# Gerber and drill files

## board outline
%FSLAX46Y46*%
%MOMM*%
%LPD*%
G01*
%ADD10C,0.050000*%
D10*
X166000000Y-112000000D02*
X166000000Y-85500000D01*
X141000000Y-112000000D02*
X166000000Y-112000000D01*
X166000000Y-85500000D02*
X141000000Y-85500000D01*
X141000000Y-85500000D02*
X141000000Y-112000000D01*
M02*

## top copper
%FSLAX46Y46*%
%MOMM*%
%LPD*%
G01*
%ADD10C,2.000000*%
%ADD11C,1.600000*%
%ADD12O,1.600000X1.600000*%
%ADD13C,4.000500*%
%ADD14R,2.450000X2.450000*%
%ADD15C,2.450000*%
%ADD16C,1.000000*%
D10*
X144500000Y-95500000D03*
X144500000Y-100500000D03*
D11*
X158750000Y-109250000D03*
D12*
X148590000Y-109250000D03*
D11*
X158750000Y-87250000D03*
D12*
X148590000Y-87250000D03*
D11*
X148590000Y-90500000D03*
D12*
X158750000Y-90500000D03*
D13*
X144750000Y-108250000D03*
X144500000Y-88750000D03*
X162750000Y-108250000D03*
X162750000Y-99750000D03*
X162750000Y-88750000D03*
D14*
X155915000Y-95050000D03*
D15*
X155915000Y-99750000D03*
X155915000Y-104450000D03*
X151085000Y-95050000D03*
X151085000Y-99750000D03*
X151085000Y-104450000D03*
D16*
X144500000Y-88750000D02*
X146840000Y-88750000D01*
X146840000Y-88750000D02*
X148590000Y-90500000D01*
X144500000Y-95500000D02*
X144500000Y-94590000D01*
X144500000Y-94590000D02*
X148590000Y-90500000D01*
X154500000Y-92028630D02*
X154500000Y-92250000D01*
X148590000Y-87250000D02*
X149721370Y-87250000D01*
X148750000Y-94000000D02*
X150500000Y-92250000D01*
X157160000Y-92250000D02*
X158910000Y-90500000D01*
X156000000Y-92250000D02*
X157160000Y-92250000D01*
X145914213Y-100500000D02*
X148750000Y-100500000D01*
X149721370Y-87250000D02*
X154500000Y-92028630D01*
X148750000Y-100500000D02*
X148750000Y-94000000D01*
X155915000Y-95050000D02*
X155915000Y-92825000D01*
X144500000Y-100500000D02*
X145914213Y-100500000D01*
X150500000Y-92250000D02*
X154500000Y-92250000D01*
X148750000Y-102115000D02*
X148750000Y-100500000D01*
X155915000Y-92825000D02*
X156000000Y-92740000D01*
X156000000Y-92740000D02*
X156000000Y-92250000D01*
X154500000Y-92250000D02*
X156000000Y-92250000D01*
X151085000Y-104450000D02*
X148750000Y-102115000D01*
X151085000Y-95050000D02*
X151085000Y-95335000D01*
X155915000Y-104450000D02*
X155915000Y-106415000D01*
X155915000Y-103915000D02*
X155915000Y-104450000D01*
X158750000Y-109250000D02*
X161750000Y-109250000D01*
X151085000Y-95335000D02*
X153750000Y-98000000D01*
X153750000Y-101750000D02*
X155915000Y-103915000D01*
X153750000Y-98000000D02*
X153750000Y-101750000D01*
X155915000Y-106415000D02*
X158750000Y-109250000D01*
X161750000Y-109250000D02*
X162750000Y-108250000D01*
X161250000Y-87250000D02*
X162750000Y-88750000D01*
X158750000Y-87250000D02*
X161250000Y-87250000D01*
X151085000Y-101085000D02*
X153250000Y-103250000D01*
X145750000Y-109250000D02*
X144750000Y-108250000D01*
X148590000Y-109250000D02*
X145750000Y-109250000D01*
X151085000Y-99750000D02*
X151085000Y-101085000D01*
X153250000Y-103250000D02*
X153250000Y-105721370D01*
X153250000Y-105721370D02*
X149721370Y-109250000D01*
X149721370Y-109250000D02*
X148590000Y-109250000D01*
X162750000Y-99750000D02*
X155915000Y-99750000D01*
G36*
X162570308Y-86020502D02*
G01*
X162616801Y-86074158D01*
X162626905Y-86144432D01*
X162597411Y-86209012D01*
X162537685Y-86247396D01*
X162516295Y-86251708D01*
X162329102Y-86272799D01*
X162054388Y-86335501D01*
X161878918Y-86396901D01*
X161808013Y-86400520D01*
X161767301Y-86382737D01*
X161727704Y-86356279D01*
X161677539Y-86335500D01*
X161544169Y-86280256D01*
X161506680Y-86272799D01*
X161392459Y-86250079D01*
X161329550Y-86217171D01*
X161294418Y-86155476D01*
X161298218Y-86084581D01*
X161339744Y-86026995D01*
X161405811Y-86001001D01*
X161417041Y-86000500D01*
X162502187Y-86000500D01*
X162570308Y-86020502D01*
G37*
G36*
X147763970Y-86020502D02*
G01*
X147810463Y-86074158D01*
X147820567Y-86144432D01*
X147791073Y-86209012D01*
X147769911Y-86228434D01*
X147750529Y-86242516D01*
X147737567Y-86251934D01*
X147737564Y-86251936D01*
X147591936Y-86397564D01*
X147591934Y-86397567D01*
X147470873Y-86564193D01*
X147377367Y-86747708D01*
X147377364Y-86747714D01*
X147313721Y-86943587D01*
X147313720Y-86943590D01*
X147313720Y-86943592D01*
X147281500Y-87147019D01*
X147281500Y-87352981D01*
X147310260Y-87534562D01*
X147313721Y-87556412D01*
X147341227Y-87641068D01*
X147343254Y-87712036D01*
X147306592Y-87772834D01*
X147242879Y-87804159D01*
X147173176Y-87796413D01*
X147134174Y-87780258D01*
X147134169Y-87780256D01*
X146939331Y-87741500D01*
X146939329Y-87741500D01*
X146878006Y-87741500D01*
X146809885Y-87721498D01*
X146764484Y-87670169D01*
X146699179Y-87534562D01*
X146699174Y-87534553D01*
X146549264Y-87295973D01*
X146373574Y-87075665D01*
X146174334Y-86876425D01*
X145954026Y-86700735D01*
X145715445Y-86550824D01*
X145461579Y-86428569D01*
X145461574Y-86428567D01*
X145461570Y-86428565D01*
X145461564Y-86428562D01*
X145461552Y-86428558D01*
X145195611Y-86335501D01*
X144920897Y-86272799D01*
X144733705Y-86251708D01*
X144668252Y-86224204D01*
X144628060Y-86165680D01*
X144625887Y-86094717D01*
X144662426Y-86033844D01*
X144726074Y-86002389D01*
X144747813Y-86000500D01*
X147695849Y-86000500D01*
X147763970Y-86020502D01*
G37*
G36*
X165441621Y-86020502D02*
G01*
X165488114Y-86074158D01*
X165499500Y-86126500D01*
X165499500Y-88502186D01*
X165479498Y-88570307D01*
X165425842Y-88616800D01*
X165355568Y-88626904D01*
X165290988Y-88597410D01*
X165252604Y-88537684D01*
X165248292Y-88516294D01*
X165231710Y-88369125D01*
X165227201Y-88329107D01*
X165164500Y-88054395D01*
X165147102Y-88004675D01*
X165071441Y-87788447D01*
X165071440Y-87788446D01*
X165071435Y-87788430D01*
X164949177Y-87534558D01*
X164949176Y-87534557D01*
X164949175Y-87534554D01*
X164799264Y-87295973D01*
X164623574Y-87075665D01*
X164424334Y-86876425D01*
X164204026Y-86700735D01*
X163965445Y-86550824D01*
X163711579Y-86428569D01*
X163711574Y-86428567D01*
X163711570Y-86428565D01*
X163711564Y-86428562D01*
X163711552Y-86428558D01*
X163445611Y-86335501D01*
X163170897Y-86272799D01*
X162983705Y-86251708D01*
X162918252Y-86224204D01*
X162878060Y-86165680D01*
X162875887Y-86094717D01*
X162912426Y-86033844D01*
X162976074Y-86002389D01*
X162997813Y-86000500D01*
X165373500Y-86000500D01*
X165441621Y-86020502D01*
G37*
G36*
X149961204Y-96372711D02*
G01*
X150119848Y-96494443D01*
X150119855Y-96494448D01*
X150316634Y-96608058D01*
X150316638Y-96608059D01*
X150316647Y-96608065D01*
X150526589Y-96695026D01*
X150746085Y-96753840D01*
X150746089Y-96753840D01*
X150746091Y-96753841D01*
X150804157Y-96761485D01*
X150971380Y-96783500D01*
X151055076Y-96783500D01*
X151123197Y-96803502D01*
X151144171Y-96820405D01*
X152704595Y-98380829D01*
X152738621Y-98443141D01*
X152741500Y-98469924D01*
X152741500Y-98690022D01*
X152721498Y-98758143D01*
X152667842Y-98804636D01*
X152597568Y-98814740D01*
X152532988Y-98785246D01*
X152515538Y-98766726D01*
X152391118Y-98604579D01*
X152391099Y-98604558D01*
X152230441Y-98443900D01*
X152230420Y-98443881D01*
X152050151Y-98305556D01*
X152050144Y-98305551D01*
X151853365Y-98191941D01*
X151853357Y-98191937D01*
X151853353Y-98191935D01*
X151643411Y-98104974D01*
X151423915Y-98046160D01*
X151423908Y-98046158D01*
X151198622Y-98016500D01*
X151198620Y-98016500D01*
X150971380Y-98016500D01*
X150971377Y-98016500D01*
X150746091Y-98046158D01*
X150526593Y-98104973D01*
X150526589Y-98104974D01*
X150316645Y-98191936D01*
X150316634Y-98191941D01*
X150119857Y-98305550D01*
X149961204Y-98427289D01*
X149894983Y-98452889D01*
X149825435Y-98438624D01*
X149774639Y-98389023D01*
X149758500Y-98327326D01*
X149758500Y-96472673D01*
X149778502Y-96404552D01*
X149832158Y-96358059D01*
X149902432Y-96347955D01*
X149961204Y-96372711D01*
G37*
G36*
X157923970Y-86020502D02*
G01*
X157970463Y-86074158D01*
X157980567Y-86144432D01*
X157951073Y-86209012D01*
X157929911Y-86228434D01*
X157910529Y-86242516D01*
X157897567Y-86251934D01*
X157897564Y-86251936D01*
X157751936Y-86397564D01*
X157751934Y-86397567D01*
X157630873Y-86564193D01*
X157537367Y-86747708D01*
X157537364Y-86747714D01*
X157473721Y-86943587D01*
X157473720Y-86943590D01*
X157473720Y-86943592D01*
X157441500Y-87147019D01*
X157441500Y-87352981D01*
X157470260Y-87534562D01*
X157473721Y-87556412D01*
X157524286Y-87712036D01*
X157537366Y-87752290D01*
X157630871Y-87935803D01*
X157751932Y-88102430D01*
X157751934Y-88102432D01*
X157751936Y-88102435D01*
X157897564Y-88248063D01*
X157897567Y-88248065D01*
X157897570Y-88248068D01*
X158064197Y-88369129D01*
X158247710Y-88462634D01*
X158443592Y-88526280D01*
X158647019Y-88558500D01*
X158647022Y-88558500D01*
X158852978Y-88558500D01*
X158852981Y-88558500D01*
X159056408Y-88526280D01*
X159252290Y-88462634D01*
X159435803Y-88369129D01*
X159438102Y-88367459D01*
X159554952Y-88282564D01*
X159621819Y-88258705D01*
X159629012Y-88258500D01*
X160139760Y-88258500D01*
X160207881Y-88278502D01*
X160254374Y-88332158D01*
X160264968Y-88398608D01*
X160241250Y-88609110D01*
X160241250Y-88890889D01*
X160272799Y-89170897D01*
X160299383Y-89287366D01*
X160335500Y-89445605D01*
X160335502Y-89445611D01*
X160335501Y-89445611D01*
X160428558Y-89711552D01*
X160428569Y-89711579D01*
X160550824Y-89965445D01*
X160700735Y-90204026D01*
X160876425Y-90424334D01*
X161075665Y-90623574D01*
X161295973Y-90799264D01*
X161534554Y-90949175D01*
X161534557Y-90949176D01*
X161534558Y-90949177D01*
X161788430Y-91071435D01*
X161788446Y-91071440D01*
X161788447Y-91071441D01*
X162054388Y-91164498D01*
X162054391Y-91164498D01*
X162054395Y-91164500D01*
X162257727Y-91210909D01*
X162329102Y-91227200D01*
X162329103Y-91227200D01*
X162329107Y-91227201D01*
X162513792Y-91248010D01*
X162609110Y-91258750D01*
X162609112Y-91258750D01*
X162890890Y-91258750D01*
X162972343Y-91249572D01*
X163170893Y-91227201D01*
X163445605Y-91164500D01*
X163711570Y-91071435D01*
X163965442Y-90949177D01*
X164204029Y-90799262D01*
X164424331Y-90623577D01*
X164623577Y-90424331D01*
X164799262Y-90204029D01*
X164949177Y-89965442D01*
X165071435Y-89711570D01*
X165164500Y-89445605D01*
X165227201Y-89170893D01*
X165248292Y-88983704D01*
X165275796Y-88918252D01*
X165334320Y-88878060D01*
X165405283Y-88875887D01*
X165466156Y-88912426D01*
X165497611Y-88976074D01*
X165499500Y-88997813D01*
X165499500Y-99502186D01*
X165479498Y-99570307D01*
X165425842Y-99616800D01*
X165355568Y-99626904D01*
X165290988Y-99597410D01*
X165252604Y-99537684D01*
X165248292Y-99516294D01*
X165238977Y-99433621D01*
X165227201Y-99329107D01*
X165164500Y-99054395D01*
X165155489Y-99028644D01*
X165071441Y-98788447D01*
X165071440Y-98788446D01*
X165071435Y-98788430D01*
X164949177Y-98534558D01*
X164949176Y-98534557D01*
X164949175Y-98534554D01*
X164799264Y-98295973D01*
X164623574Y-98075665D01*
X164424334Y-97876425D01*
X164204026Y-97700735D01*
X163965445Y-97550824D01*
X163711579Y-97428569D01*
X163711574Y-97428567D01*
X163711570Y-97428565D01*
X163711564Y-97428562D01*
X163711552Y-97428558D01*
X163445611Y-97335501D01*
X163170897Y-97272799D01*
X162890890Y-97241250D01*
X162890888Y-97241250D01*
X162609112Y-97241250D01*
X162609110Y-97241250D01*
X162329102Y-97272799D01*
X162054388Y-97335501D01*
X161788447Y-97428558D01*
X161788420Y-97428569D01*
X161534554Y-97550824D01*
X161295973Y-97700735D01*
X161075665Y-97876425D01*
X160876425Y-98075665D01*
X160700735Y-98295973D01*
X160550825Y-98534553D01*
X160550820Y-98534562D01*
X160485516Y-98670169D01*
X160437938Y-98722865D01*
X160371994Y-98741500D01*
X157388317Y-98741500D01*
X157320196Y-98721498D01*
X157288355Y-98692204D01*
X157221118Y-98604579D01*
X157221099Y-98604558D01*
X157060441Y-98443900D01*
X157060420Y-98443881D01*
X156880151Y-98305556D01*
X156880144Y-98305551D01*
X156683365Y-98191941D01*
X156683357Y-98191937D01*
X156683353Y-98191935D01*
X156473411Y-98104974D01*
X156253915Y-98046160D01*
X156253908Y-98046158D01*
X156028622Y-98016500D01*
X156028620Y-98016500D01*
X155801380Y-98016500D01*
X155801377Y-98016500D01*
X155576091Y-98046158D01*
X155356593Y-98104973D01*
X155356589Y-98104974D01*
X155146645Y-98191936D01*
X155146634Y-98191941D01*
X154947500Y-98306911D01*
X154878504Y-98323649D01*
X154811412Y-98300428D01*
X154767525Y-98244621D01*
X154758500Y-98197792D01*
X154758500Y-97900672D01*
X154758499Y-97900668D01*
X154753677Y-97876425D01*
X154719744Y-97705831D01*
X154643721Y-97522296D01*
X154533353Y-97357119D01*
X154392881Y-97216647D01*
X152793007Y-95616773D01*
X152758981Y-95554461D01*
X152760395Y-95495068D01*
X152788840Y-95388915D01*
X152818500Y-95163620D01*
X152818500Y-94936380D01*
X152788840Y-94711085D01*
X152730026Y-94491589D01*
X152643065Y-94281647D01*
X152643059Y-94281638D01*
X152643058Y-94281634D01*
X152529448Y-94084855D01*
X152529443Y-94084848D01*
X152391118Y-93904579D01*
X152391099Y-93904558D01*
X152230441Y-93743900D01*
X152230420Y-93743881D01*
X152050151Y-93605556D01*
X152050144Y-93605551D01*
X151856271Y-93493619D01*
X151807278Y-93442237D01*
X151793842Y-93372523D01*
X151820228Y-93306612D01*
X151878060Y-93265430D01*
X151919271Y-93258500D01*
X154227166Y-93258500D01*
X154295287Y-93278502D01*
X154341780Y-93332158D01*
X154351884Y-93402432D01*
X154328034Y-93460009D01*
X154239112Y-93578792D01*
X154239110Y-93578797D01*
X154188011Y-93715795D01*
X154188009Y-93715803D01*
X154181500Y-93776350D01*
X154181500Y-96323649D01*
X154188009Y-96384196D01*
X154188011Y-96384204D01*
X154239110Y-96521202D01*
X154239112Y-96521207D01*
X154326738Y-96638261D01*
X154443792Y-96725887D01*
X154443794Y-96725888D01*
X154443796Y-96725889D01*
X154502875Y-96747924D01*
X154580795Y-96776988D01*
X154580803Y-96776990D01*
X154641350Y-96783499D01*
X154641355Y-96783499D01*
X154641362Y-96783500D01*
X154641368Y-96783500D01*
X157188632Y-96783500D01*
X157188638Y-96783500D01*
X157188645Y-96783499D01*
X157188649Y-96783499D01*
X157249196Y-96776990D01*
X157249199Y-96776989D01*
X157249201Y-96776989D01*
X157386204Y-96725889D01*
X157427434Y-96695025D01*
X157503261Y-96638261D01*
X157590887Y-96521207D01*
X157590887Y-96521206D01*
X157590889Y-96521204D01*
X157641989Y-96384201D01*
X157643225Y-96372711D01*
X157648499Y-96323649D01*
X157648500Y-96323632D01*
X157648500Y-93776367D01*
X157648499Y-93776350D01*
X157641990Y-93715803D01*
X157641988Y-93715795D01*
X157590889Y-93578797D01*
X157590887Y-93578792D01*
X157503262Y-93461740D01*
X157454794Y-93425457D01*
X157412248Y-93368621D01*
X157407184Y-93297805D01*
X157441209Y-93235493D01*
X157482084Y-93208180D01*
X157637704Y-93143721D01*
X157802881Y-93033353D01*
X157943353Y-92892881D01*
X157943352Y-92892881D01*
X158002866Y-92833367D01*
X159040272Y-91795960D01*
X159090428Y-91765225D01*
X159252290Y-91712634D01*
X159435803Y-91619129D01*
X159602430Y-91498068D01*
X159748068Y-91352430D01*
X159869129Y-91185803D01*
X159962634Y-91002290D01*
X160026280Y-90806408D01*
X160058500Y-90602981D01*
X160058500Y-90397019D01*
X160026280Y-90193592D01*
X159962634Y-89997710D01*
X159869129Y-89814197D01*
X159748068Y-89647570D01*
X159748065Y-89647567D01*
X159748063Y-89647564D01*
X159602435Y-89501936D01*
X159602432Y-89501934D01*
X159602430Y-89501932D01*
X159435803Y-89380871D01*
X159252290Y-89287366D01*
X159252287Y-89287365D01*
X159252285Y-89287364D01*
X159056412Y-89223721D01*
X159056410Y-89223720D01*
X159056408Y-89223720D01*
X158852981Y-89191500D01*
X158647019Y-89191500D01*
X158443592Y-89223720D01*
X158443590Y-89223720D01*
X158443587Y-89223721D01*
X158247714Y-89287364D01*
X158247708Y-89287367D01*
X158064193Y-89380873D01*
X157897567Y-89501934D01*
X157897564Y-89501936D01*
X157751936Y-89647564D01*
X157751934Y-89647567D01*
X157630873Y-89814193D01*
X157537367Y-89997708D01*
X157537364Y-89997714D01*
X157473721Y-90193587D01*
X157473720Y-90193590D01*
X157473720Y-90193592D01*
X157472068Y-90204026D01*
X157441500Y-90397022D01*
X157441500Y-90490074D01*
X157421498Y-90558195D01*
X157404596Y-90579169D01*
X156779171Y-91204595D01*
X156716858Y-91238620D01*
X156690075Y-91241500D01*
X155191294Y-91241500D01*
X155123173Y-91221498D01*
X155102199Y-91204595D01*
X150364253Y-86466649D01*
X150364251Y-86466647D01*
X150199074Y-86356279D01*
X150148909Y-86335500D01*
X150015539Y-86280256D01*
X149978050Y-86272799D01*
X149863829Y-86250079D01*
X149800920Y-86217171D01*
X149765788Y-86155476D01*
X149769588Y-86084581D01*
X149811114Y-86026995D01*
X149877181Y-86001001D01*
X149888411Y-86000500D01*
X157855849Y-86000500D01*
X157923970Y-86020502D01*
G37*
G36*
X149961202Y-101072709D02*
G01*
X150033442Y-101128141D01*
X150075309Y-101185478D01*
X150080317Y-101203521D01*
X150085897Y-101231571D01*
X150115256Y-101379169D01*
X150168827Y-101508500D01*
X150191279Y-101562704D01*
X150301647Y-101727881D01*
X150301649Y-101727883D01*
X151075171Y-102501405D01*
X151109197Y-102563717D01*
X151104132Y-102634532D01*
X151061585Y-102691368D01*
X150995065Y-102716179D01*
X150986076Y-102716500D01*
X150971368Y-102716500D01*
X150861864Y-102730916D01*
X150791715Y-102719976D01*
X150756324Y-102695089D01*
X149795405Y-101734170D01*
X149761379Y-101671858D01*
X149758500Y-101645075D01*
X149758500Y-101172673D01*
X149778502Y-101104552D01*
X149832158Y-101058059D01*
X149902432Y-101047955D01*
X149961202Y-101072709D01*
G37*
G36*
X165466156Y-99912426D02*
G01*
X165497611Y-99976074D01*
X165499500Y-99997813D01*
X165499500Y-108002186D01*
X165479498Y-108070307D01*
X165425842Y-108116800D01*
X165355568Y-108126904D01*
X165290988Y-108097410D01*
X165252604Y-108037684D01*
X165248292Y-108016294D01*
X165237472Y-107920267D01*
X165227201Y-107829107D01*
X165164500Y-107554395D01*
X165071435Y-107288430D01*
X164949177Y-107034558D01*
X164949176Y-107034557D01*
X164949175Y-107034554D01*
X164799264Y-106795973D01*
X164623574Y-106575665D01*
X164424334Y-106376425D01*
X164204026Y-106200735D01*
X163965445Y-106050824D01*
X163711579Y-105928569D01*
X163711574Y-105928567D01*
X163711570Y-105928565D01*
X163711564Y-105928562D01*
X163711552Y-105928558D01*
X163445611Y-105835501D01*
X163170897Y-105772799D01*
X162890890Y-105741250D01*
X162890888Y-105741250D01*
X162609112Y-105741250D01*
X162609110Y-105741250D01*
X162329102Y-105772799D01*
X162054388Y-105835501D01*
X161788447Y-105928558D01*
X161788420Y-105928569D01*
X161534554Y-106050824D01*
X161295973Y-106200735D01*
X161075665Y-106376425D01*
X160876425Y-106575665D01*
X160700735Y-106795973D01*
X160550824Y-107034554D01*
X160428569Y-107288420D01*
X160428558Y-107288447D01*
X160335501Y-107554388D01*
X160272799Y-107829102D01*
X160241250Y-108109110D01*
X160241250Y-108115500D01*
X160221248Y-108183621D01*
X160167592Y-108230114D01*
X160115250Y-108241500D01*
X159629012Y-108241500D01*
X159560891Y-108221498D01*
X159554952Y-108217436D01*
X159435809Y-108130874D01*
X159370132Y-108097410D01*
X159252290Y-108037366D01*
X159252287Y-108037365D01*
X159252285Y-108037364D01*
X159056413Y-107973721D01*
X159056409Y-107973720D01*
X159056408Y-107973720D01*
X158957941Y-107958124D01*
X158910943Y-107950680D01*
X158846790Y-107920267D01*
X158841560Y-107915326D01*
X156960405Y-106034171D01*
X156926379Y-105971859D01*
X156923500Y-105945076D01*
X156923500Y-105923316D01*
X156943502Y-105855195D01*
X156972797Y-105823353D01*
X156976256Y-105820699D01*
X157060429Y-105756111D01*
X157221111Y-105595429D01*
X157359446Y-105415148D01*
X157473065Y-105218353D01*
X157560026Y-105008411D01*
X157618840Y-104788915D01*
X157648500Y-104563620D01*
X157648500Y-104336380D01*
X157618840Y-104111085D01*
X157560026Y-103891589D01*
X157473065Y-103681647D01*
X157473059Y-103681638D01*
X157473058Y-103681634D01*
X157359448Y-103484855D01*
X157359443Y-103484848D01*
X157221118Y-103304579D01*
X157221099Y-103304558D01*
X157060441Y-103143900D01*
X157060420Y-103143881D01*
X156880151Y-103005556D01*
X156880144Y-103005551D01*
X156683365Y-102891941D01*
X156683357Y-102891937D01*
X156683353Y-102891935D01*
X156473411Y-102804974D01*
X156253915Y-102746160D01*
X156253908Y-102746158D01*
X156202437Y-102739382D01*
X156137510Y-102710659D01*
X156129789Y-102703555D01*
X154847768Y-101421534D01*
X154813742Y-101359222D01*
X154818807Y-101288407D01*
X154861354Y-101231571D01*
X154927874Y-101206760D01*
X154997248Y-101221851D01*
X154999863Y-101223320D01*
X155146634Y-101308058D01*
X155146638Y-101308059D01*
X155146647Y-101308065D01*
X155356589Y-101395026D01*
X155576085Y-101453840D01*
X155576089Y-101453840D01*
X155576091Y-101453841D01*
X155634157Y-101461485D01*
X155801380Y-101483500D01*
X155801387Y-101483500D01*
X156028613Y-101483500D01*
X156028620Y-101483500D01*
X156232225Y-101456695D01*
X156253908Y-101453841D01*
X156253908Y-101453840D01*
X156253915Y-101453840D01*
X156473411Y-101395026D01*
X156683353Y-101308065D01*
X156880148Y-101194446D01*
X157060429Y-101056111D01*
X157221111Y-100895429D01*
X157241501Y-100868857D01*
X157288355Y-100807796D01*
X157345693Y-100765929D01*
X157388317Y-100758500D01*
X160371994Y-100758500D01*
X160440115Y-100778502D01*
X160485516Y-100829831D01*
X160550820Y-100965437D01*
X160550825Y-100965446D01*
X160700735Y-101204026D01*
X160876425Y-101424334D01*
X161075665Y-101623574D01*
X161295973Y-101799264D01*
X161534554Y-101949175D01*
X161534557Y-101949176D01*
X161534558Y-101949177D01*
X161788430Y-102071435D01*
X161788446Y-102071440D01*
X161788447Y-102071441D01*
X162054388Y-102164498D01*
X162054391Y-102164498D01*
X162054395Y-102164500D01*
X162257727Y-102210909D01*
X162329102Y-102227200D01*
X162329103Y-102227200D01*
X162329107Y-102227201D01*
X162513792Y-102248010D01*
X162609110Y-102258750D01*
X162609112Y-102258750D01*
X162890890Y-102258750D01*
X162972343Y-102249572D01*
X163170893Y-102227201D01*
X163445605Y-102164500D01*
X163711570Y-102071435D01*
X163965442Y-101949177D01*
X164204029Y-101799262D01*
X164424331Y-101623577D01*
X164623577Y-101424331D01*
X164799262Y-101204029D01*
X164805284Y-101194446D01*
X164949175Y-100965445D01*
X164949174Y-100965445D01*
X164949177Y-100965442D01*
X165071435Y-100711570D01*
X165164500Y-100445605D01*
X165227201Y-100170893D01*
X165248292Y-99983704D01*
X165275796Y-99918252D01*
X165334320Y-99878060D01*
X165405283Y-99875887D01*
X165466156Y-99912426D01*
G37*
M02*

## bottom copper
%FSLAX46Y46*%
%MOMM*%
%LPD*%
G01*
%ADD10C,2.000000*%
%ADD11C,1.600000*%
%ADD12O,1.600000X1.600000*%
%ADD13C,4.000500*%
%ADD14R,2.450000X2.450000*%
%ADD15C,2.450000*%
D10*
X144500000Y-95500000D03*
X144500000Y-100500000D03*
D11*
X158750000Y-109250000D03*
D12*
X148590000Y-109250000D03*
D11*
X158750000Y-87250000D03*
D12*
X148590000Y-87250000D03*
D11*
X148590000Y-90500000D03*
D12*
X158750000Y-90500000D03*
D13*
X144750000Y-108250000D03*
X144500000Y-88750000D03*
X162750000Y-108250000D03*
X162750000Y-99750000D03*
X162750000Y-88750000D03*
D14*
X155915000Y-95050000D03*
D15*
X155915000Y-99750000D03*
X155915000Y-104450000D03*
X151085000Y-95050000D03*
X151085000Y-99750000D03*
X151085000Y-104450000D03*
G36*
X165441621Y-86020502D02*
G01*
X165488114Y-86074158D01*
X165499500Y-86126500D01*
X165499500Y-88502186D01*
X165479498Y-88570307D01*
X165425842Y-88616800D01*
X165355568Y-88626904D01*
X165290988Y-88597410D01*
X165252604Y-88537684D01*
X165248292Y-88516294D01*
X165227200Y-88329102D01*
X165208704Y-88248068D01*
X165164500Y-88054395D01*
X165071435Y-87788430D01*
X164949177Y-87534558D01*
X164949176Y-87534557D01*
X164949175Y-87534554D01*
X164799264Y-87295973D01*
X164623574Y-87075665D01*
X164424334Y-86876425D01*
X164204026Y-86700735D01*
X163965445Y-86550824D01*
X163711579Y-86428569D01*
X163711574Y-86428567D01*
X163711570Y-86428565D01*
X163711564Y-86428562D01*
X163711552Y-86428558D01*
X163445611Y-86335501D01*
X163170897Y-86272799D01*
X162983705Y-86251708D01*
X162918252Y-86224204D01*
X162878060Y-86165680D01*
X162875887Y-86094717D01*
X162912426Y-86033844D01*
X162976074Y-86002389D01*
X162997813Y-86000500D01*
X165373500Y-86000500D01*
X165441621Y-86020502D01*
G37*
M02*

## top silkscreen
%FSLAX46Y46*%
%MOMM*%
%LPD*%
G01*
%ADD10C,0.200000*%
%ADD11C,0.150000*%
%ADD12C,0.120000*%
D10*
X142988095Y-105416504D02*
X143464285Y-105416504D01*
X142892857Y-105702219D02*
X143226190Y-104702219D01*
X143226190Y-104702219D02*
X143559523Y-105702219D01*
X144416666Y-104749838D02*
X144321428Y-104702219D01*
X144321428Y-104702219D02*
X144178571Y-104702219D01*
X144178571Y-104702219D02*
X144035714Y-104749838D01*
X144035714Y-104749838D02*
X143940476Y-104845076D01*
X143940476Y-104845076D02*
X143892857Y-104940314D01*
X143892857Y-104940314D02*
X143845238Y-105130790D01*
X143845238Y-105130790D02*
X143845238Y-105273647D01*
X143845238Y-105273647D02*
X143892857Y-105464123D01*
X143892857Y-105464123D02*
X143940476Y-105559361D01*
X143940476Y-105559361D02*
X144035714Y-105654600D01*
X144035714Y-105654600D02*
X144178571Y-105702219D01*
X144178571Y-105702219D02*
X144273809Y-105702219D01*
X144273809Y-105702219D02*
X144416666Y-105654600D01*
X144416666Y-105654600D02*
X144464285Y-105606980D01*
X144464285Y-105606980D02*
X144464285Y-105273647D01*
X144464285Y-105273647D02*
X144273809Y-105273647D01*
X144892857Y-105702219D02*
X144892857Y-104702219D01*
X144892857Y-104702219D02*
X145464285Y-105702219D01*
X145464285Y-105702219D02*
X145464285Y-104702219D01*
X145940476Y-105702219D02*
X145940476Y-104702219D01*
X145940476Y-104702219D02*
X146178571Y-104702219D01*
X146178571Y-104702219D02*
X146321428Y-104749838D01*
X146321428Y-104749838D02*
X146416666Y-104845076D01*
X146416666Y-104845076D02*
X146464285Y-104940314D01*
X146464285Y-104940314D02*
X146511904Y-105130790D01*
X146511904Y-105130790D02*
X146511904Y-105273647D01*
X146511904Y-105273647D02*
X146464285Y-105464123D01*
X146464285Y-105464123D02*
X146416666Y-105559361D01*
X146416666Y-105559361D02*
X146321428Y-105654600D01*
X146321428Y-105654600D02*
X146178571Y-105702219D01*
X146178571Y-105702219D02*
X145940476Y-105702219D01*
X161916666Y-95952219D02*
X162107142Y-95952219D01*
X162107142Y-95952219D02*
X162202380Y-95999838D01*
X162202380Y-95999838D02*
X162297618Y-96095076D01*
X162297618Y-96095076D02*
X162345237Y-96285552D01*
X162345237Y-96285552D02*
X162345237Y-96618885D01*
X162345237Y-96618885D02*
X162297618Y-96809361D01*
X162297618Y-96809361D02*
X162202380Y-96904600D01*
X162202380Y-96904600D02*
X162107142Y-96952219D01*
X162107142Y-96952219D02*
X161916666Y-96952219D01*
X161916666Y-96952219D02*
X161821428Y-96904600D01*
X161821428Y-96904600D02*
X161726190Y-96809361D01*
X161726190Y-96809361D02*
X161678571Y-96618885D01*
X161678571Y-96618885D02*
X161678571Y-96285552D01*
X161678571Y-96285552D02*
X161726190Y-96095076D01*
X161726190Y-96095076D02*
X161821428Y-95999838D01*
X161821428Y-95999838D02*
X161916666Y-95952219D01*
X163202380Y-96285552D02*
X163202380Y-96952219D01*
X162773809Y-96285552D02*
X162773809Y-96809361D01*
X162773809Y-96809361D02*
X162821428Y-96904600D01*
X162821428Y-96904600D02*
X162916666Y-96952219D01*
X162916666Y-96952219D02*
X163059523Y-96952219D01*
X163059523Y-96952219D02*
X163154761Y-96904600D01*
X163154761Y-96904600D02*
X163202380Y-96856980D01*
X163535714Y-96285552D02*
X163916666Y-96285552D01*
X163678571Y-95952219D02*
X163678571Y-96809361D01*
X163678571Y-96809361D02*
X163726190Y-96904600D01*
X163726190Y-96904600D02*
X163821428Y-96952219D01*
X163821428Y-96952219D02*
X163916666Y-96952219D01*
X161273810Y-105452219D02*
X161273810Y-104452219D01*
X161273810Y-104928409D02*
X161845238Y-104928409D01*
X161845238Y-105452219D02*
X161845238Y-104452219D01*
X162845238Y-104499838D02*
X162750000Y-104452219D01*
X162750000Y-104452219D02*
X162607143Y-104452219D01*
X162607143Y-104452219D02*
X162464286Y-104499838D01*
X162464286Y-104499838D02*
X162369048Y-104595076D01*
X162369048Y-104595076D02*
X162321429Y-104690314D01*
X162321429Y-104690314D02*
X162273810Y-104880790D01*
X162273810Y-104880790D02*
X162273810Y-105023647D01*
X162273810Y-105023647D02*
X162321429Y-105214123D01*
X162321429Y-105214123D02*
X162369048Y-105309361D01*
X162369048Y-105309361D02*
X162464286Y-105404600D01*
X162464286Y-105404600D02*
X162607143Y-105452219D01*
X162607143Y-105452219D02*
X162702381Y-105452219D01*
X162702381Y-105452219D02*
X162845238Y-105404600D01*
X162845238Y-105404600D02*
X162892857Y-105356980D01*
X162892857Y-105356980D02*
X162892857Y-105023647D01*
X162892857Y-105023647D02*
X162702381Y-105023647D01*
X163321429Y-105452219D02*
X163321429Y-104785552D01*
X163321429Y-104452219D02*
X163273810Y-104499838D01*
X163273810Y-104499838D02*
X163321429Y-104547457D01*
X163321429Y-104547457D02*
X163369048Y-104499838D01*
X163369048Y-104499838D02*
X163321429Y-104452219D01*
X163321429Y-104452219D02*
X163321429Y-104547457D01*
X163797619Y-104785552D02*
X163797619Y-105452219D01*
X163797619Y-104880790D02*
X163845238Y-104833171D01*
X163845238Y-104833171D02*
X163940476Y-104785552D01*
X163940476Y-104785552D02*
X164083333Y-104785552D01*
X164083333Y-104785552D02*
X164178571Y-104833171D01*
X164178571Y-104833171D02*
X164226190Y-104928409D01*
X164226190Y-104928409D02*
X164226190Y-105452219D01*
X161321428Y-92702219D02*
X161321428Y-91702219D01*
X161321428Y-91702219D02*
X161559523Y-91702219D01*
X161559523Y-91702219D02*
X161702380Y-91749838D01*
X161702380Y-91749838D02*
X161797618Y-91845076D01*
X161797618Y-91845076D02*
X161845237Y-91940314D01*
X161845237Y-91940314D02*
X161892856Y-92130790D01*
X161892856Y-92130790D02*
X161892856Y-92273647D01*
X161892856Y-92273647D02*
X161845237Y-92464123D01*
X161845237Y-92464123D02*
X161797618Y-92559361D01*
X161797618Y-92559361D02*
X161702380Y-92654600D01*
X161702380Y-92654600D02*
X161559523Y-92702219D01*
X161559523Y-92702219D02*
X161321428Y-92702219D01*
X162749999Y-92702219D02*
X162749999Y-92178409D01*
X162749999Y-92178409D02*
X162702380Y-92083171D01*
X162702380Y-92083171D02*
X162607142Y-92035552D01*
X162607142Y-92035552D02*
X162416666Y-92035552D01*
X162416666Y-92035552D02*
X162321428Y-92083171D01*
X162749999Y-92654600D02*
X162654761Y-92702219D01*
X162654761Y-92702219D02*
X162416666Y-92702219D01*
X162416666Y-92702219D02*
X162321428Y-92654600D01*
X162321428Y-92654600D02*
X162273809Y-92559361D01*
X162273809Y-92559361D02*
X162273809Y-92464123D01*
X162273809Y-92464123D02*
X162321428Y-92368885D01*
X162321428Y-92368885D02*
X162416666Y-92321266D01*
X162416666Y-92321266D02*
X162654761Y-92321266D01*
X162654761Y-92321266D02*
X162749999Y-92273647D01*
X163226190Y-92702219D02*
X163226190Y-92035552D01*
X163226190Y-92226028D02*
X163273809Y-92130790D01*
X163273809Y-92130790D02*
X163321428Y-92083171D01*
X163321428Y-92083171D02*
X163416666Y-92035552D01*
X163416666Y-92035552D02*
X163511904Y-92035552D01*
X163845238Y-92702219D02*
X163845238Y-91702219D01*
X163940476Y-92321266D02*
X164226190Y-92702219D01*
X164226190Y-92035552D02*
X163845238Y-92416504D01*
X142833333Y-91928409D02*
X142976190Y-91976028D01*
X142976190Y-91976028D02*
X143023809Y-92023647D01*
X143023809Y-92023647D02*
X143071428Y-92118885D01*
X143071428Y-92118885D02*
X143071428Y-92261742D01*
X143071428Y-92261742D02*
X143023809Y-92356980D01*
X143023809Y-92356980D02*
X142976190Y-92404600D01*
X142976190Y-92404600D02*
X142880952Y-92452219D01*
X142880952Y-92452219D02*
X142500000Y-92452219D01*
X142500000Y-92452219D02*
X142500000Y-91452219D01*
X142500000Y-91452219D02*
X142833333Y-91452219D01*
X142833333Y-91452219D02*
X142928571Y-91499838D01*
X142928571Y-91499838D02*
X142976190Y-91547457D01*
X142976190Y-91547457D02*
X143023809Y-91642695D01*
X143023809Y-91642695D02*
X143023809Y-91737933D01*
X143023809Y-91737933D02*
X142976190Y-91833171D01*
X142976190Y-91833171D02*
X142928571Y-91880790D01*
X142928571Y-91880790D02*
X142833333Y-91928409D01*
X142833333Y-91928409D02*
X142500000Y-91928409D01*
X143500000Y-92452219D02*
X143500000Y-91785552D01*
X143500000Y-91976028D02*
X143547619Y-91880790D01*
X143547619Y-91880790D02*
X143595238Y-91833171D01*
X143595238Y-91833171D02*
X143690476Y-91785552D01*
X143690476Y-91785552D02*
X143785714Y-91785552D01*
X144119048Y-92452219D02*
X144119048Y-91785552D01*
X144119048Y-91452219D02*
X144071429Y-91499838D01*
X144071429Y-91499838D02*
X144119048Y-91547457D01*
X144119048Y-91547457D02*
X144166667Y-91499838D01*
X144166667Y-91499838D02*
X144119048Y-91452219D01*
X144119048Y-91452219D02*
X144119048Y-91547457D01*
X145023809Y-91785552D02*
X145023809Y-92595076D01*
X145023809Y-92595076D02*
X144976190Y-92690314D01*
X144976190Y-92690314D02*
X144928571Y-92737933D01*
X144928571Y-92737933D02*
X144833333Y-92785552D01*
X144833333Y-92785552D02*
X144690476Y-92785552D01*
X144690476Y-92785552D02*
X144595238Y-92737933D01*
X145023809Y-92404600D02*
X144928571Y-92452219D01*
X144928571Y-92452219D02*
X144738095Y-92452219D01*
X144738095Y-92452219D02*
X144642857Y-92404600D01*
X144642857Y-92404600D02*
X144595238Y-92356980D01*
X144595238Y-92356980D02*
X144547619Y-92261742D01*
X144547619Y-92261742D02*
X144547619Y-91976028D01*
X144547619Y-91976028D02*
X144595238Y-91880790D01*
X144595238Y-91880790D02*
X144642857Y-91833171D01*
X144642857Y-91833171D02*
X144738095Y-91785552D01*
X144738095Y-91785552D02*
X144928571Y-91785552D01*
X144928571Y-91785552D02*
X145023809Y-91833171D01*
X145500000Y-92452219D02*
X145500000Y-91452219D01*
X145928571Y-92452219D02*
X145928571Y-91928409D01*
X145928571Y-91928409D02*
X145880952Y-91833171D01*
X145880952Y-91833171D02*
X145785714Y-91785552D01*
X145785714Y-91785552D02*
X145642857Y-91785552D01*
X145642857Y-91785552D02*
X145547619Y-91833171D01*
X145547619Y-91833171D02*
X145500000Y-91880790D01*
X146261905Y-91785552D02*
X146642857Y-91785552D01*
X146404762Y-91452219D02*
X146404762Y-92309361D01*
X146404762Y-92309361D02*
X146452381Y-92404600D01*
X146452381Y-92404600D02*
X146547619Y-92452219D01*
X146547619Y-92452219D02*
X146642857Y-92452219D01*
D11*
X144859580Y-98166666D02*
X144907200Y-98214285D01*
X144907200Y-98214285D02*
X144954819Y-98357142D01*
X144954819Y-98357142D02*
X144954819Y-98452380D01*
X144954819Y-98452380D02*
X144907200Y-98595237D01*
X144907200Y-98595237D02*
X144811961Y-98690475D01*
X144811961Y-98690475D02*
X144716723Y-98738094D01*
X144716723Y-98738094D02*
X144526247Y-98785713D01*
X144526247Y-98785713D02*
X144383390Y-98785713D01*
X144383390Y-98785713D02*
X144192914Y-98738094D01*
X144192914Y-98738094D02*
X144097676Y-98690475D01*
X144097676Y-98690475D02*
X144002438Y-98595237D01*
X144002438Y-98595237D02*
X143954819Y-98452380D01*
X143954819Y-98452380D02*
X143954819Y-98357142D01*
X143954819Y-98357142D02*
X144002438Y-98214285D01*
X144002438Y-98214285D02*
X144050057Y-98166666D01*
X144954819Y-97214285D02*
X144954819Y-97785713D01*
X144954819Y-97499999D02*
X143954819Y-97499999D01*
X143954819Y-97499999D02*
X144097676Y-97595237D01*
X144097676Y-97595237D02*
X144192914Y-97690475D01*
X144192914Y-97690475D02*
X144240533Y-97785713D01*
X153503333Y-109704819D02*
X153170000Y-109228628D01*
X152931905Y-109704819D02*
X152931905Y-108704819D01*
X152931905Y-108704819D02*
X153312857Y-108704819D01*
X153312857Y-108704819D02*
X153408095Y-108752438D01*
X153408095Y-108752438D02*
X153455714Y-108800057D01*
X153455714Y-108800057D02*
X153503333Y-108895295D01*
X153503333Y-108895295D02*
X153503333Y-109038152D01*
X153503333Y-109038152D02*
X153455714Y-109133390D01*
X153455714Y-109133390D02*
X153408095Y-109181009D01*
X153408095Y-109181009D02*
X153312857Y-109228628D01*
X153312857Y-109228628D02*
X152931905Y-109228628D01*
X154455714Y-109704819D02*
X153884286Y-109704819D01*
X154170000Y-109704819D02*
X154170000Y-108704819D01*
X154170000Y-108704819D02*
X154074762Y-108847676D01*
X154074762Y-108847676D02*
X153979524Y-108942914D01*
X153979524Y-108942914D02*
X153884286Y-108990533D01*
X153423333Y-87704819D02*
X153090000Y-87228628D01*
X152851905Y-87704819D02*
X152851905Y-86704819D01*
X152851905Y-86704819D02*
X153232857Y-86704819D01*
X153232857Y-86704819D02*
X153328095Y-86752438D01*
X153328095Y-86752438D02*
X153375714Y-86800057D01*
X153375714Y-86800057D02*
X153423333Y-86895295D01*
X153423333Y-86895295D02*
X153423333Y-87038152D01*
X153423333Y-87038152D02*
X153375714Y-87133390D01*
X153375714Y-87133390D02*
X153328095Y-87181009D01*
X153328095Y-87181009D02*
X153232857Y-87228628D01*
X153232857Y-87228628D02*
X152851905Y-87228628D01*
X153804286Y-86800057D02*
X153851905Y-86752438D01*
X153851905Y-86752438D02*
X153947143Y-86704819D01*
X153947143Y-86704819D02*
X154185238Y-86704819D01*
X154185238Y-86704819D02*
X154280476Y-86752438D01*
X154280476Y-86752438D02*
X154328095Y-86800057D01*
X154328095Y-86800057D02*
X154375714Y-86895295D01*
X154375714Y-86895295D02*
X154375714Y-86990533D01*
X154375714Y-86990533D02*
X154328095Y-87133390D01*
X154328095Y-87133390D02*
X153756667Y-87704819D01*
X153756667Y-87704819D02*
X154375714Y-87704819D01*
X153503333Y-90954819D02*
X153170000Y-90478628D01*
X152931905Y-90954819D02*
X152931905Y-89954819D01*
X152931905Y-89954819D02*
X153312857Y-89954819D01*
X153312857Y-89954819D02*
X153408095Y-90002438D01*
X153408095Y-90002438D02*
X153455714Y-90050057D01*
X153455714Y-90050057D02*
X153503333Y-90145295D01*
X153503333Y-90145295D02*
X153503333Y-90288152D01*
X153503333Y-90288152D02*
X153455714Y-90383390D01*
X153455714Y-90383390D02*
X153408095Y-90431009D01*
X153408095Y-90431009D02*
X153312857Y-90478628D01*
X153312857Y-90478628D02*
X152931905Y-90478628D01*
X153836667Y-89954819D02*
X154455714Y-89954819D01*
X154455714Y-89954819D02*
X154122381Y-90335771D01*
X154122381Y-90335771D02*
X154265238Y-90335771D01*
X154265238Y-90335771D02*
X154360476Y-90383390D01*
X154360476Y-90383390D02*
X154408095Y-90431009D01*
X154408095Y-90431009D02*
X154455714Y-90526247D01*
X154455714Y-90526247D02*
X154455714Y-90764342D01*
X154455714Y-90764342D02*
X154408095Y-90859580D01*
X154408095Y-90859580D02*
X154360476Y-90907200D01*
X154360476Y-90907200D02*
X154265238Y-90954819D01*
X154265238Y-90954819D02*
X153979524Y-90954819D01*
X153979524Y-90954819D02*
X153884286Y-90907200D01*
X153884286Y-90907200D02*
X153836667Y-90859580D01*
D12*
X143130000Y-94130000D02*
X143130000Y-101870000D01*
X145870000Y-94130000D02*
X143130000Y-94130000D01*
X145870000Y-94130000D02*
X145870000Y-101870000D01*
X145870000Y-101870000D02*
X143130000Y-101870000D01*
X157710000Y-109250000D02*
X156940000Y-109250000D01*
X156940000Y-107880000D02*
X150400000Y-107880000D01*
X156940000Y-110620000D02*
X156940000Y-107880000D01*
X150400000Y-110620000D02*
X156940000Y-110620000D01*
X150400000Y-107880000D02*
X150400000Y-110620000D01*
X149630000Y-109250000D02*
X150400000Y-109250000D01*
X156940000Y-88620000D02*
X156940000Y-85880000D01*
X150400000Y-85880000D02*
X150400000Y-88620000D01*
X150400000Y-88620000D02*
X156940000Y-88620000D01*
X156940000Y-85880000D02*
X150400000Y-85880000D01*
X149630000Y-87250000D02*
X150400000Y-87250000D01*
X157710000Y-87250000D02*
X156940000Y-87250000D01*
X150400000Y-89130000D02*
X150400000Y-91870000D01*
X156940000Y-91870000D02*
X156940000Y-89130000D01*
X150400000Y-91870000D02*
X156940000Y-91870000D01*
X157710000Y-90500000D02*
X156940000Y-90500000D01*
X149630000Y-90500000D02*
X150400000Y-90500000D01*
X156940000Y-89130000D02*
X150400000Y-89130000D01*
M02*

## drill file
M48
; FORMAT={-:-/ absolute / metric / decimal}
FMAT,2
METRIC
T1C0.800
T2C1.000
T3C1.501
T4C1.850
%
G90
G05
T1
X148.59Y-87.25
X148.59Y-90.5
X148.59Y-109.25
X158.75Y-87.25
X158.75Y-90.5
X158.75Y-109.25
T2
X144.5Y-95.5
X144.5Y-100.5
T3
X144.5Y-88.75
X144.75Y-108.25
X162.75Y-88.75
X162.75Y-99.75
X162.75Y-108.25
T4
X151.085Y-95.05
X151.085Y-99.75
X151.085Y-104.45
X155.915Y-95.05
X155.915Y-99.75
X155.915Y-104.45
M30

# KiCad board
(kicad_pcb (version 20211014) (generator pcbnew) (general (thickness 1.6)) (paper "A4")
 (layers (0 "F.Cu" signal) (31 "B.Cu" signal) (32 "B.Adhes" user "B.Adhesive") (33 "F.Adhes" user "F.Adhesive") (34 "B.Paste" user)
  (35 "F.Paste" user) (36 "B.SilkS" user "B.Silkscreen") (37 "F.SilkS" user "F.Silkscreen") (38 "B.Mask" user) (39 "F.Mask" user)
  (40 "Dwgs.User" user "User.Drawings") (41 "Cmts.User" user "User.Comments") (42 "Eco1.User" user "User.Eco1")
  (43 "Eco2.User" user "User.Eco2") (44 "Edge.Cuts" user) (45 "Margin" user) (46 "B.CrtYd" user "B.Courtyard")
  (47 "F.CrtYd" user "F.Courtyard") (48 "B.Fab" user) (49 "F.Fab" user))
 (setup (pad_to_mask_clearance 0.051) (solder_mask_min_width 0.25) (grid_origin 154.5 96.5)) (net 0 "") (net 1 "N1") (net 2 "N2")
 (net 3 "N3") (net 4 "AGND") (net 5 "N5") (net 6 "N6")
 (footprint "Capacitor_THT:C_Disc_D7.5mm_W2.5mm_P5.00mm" (layer "F.Cu") (at 144.5 95.5 -90)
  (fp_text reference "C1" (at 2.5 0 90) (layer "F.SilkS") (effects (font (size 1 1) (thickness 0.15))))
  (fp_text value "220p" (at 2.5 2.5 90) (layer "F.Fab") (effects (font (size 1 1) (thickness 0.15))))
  (fp_line (start -1.37 1.37) (end 6.37 1.37) (layer "F.SilkS") (width 0.12))
  (fp_line (start -1.37 -1.37) (end -1.37 1.37) (layer "F.SilkS") (width 0.12))
  (fp_line (start -1.37 -1.37) (end 6.37 -1.37) (layer "F.SilkS") (width 0.12))
  (fp_line (start 6.37 -1.37) (end 6.37 1.37) (layer "F.SilkS") (width 0.12))
  (pad "1" thru_hole circle locked (at 0 0 270) (size 2 2) (drill 1) (layers *.Cu *.Mask) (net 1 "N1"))
  (pad "2" thru_hole circle locked (at 5 0 270) (size 2 2) (drill 1) (layers *.Cu *.Mask) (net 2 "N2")))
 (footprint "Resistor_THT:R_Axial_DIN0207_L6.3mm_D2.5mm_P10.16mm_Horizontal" (layer "F.Cu") (at 158.75 109.25 180)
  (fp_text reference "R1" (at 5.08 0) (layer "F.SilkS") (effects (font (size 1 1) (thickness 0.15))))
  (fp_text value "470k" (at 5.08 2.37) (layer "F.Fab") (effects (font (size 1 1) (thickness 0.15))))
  (fp_line (start 1.04 0) (end 1.81 0) (layer "F.SilkS") (width 0.12))
  (fp_line (start 1.81 1.37) (end 8.35 1.37) (layer "F.SilkS") (width 0.12))
  (fp_line (start 1.81 -1.37) (end 1.81 1.37) (layer "F.SilkS") (width 0.12))
  (fp_line (start 8.35 -1.37) (end 1.81 -1.37) (layer "F.SilkS") (width 0.12))
  (fp_line (start 8.35 1.37) (end 8.35 -1.37) (layer "F.SilkS") (width 0.12))
  (fp_line (start 9.12 0) (end 8.35 0) (layer "F.SilkS") (width 0.12))
  (pad "1" thru_hole circle locked (at 0 0 180) (size 1.6 1.6) (drill 0.8) (layers *.Cu *.Mask) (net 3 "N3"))
  (pad "2" thru_hole oval locked (at 10.16 0 180) (size 1.6 1.6) (drill 0.8) (layers *.Cu *.Mask) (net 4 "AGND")))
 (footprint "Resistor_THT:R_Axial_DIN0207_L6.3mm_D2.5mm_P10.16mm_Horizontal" (layer "F.Cu") (at 158.75 87.25 180)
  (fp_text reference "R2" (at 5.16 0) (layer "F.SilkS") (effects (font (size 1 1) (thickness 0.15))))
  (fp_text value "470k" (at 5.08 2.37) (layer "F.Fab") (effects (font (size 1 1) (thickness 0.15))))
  (fp_line (start 1.81 -1.37) (end 1.81 1.37) (layer "F.SilkS") (width 0.12))
  (fp_line (start 8.35 1.37) (end 8.35 -1.37) (layer "F.SilkS") (width 0.12))
  (fp_line (start 8.35 -1.37) (end 1.81 -1.37) (layer "F.SilkS") (width 0.12))
  (fp_line (start 1.81 1.37) (end 8.35 1.37) (layer "F.SilkS") (width 0.12))
  (fp_line (start 9.12 0) (end 8.35 0) (layer "F.SilkS") (width 0.12))
  (fp_line (start 1.04 0) (end 1.81 0) (layer "F.SilkS") (width 0.12))
  (pad "1" thru_hole circle locked (at 0 0 180) (size 1.6 1.6) (drill 0.8) (layers *.Cu *.Mask) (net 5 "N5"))
  (pad "2" thru_hole oval locked (at 10.16 0 180) (size 1.6 1.6) (drill 0.8) (layers *.Cu *.Mask) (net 2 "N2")))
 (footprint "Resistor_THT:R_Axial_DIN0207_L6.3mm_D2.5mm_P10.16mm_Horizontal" (layer "F.Cu") (at 148.59 90.5)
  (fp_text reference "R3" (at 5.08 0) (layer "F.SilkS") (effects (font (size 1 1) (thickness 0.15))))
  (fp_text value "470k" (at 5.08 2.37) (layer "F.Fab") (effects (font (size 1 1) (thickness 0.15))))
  (fp_line (start 1.81 -1.37) (end 1.81 1.37) (layer "F.SilkS") (width 0.12))
  (fp_line (start 8.35 1.37) (end 8.35 -1.37) (layer "F.SilkS") (width 0.12))
  (fp_line (start 1.81 1.37) (end 8.35 1.37) (layer "F.SilkS") (width 0.12))
  (fp_line (start 9.12 0) (end 8.35 0) (layer "F.SilkS") (width 0.12))
  (fp_line (start 1.04 0) (end 1.81 0) (layer "F.SilkS") (width 0.12))
  (fp_line (start 8.35 -1.37) (end 1.81 -1.37) (layer "F.SilkS") (width 0.12))
  (pad "1" thru_hole circle locked (at 0 0) (size 1.6 1.6) (drill 0.8) (layers *.Cu *.Mask) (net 1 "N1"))
  (pad "2" thru_hole oval locked (at 10.16 0) (size 1.6 1.6) (drill 0.8) (layers *.Cu *.Mask) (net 2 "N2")))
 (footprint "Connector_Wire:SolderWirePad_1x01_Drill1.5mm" (layer "F.Cu") (at 144.75 108.25)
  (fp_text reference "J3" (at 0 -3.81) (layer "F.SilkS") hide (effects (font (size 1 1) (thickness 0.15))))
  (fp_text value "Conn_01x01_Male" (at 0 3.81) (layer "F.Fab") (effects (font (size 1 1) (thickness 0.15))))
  (pad "1" thru_hole circle locked (at 0 0) (size 4.0005 4.0005) (drill 1.50114) (layers *.Cu *.Mask) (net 4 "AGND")))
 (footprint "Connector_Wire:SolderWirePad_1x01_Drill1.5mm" (layer "F.Cu") (at 144.5 88.75 180)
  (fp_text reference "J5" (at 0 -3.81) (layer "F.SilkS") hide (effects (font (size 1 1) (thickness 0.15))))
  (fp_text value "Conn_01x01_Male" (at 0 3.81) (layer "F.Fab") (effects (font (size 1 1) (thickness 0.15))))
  (pad "1" thru_hole circle locked (at 0 0 180) (size 4.0005 4.0005) (drill 1.50114) (layers *.Cu *.Mask) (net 1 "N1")))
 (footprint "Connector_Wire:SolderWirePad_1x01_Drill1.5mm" (layer "F.Cu") (at 162.75 108.25)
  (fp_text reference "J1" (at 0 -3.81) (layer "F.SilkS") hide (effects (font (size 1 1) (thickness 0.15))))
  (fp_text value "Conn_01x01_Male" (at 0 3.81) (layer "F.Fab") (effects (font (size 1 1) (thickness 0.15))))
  (pad "1" thru_hole circle locked (at 0 0) (size 4.0005 4.0005) (drill 1.50114) (layers *.Cu *.Mask) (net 3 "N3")))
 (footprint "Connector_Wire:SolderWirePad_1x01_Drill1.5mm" (layer "F.Cu") (at 162.75 99.75 180)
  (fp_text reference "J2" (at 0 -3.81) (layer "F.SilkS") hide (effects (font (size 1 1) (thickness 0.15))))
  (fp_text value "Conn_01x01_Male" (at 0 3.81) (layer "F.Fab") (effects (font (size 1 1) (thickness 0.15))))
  (pad "1" thru_hole circle locked (at 0 0 180) (size 4.0005 4.0005) (drill 1.50114) (layers *.Cu *.Mask) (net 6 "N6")))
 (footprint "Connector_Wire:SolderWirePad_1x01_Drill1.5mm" (layer "F.Cu") (at 162.75 88.75 180)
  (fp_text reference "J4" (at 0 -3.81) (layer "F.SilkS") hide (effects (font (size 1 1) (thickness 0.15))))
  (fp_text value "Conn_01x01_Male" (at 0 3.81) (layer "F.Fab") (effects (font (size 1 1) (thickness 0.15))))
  (pad "1" thru_hole circle locked (at 0 0 180) (size 4.0005 4.0005) (drill 1.50114) (layers *.Cu *.Mask) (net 5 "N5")))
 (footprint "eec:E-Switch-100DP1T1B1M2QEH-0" (layer "B.Cu") (at 153.5 99.75 -90)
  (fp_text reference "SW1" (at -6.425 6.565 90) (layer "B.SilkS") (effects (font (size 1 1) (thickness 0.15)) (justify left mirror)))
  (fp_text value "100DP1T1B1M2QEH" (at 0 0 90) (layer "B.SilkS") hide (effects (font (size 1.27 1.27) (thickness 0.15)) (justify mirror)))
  (pad "1" thru_hole rect locked (at -4.7 -2.415 270) (size 2.45 2.45) (drill 1.85) (layers *.Cu *.Mask) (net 2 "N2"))
  (pad "2" thru_hole circle locked (at 0 -2.415 270) (size 2.45 2.45) (drill 1.85) (layers *.Cu *.Mask) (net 6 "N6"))
  (pad "3" thru_hole circle locked (at 4.7 -2.415 270) (size 2.45 2.45) (drill 1.85) (layers *.Cu *.Mask) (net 3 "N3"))
  (pad "4" thru_hole circle locked (at -4.7 2.415 270) (size 2.45 2.45) (drill 1.85) (layers *.Cu *.Mask) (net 3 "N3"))
  (pad "5" thru_hole circle locked (at 0 2.415 270) (size 2.45 2.45) (drill 1.85) (layers *.Cu *.Mask) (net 4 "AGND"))
  (pad "6" thru_hole circle locked (at 4.7 2.415 270) (size 2.45 2.45) (drill 1.85) (layers *.Cu *.Mask) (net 2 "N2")))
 (gr_line (start 166 112) (end 166 85.5) (layer "Edge.Cuts") (width 0.05))
 (gr_line (start 141 112) (end 166 112) (layer "Edge.Cuts") (width 0.05))
 (gr_line (start 166 85.5) (end 141 85.5) (layer "Edge.Cuts") (width 0.05))
 (gr_line (start 141 85.5) (end 141 112) (layer "Edge.Cuts") (width 0.05))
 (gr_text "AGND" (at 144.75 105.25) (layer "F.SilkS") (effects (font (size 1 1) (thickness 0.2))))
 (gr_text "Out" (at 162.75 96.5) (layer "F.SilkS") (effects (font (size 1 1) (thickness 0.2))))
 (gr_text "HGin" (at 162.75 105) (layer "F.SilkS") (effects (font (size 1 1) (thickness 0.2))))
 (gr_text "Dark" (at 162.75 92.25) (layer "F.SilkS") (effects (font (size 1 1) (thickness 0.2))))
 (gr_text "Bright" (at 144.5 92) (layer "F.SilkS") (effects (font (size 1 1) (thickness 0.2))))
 (segment (start 144.5 88.75) (end 146.84 88.75) (width 1) (layer "F.Cu") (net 1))
 (segment (start 146.84 88.75) (end 148.59 90.5) (width 1) (layer "F.Cu") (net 1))
 (segment (start 144.5 95.5) (end 144.5 94.59) (width 1) (layer "F.Cu") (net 1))
 (segment (start 144.5 94.59) (end 148.59 90.5) (width 1) (layer "F.Cu") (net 1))
 (segment (start 154.5 92.02863) (end 154.5 92.25) (width 1) (layer "F.Cu") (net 2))
 (segment (start 148.59 87.25) (end 149.72137 87.25) (width 1) (layer "F.Cu") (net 2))
 (segment (start 148.75 94) (end 150.5 92.25) (width 1) (layer "F.Cu") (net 2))
 (segment (start 157.16 92.25) (end 158.91 90.5) (width 1) (layer "F.Cu") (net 2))
 (segment (start 156 92.25) (end 157.16 92.25) (width 1) (layer "F.Cu") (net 2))
 (segment (start 145.914213 100.5) (end 148.75 100.5) (width 1) (layer "F.Cu") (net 2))
 (segment (start 149.72137 87.25) (end 154.5 92.02863) (width 1) (layer "F.Cu") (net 2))
 (segment (start 148.75 100.5) (end 148.75 94) (width 1) (layer "F.Cu") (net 2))
 (segment (start 155.915 95.05) (end 155.915 92.825) (width 1) (layer "F.Cu") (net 2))
 (segment (start 144.5 100.5) (end 145.914213 100.5) (width 1) (layer "F.Cu") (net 2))
 (segment (start 150.5 92.25) (end 154.5 92.25) (width 1) (layer "F.Cu") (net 2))
 (segment (start 148.75 102.115) (end 148.75 100.5) (width 1) (layer "F.Cu") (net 2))
 (segment (start 155.915 92.825) (end 156 92.74) (width 1) (layer "F.Cu") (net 2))
 (segment (start 156 92.74) (end 156 92.25) (width 1) (layer "F.Cu") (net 2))
 (segment (start 154.5 92.25) (end 156 92.25) (width 1) (layer "F.Cu") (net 2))
 (segment (start 151.085 104.45) (end 148.75 102.115) (width 1) (layer "F.Cu") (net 2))
 (segment (start 151.085 95.05) (end 151.085 95.335) (width 1) (layer "F.Cu") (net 3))
 (segment (start 155.915 104.45) (end 155.915 106.415) (width 1) (layer "F.Cu") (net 3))
 (segment (start 155.915 103.915) (end 155.915 104.45) (width 1) (layer "F.Cu") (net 3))
 (segment (start 158.75 109.25) (end 161.75 109.25) (width 1) (layer "F.Cu") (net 3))
 (segment (start 151.085 95.335) (end 153.75 98) (width 1) (layer "F.Cu") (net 3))
 (segment (start 153.75 101.75) (end 155.915 103.915) (width 1) (layer "F.Cu") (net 3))
 (segment (start 153.75 98) (end 153.75 101.75) (width 1) (layer "F.Cu") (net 3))
 (segment (start 155.915 106.415) (end 158.75 109.25) (width 1) (layer "F.Cu") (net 3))
 (segment (start 161.75 109.25) (end 162.75 108.25) (width 1) (layer "F.Cu") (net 3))
 (segment (start 161.25 87.25) (end 162.75 88.75) (width 1) (layer "F.Cu") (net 5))
 (segment (start 158.75 87.25) (end 161.25 87.25) (width 1) (layer "F.Cu") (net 5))
 (segment (start 151.085 101.085) (end 153.25 103.25) (width 1) (layer "F.Cu") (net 4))
 (segment (start 145.75 109.25) (end 144.75 108.25) (width 1) (layer "F.Cu") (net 4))
 (segment (start 148.59 109.25) (end 145.75 109.25) (width 1) (layer "F.Cu") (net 4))
 (segment (start 151.085 99.75) (end 151.085 101.085) (width 1) (layer "F.Cu") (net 4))
 (segment (start 153.25 103.25) (end 153.25 105.72137) (width 1) (layer "F.Cu") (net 4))
 (segment (start 153.25 105.72137) (end 149.72137 109.25) (width 1) (layer "F.Cu") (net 4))
 (segment (start 149.72137 109.25) (end 148.59 109.25) (width 1) (layer "F.Cu") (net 4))
 (segment (start 162.75 99.75) (end 155.915 99.75) (width 1) (layer "F.Cu") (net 6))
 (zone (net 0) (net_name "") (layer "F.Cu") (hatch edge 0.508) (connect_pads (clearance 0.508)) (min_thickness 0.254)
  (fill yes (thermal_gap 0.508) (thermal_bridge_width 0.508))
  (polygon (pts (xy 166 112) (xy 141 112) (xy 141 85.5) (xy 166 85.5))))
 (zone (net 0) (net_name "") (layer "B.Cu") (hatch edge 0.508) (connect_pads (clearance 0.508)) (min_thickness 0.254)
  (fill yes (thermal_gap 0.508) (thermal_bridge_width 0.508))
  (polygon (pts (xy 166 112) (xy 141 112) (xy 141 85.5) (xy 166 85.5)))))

